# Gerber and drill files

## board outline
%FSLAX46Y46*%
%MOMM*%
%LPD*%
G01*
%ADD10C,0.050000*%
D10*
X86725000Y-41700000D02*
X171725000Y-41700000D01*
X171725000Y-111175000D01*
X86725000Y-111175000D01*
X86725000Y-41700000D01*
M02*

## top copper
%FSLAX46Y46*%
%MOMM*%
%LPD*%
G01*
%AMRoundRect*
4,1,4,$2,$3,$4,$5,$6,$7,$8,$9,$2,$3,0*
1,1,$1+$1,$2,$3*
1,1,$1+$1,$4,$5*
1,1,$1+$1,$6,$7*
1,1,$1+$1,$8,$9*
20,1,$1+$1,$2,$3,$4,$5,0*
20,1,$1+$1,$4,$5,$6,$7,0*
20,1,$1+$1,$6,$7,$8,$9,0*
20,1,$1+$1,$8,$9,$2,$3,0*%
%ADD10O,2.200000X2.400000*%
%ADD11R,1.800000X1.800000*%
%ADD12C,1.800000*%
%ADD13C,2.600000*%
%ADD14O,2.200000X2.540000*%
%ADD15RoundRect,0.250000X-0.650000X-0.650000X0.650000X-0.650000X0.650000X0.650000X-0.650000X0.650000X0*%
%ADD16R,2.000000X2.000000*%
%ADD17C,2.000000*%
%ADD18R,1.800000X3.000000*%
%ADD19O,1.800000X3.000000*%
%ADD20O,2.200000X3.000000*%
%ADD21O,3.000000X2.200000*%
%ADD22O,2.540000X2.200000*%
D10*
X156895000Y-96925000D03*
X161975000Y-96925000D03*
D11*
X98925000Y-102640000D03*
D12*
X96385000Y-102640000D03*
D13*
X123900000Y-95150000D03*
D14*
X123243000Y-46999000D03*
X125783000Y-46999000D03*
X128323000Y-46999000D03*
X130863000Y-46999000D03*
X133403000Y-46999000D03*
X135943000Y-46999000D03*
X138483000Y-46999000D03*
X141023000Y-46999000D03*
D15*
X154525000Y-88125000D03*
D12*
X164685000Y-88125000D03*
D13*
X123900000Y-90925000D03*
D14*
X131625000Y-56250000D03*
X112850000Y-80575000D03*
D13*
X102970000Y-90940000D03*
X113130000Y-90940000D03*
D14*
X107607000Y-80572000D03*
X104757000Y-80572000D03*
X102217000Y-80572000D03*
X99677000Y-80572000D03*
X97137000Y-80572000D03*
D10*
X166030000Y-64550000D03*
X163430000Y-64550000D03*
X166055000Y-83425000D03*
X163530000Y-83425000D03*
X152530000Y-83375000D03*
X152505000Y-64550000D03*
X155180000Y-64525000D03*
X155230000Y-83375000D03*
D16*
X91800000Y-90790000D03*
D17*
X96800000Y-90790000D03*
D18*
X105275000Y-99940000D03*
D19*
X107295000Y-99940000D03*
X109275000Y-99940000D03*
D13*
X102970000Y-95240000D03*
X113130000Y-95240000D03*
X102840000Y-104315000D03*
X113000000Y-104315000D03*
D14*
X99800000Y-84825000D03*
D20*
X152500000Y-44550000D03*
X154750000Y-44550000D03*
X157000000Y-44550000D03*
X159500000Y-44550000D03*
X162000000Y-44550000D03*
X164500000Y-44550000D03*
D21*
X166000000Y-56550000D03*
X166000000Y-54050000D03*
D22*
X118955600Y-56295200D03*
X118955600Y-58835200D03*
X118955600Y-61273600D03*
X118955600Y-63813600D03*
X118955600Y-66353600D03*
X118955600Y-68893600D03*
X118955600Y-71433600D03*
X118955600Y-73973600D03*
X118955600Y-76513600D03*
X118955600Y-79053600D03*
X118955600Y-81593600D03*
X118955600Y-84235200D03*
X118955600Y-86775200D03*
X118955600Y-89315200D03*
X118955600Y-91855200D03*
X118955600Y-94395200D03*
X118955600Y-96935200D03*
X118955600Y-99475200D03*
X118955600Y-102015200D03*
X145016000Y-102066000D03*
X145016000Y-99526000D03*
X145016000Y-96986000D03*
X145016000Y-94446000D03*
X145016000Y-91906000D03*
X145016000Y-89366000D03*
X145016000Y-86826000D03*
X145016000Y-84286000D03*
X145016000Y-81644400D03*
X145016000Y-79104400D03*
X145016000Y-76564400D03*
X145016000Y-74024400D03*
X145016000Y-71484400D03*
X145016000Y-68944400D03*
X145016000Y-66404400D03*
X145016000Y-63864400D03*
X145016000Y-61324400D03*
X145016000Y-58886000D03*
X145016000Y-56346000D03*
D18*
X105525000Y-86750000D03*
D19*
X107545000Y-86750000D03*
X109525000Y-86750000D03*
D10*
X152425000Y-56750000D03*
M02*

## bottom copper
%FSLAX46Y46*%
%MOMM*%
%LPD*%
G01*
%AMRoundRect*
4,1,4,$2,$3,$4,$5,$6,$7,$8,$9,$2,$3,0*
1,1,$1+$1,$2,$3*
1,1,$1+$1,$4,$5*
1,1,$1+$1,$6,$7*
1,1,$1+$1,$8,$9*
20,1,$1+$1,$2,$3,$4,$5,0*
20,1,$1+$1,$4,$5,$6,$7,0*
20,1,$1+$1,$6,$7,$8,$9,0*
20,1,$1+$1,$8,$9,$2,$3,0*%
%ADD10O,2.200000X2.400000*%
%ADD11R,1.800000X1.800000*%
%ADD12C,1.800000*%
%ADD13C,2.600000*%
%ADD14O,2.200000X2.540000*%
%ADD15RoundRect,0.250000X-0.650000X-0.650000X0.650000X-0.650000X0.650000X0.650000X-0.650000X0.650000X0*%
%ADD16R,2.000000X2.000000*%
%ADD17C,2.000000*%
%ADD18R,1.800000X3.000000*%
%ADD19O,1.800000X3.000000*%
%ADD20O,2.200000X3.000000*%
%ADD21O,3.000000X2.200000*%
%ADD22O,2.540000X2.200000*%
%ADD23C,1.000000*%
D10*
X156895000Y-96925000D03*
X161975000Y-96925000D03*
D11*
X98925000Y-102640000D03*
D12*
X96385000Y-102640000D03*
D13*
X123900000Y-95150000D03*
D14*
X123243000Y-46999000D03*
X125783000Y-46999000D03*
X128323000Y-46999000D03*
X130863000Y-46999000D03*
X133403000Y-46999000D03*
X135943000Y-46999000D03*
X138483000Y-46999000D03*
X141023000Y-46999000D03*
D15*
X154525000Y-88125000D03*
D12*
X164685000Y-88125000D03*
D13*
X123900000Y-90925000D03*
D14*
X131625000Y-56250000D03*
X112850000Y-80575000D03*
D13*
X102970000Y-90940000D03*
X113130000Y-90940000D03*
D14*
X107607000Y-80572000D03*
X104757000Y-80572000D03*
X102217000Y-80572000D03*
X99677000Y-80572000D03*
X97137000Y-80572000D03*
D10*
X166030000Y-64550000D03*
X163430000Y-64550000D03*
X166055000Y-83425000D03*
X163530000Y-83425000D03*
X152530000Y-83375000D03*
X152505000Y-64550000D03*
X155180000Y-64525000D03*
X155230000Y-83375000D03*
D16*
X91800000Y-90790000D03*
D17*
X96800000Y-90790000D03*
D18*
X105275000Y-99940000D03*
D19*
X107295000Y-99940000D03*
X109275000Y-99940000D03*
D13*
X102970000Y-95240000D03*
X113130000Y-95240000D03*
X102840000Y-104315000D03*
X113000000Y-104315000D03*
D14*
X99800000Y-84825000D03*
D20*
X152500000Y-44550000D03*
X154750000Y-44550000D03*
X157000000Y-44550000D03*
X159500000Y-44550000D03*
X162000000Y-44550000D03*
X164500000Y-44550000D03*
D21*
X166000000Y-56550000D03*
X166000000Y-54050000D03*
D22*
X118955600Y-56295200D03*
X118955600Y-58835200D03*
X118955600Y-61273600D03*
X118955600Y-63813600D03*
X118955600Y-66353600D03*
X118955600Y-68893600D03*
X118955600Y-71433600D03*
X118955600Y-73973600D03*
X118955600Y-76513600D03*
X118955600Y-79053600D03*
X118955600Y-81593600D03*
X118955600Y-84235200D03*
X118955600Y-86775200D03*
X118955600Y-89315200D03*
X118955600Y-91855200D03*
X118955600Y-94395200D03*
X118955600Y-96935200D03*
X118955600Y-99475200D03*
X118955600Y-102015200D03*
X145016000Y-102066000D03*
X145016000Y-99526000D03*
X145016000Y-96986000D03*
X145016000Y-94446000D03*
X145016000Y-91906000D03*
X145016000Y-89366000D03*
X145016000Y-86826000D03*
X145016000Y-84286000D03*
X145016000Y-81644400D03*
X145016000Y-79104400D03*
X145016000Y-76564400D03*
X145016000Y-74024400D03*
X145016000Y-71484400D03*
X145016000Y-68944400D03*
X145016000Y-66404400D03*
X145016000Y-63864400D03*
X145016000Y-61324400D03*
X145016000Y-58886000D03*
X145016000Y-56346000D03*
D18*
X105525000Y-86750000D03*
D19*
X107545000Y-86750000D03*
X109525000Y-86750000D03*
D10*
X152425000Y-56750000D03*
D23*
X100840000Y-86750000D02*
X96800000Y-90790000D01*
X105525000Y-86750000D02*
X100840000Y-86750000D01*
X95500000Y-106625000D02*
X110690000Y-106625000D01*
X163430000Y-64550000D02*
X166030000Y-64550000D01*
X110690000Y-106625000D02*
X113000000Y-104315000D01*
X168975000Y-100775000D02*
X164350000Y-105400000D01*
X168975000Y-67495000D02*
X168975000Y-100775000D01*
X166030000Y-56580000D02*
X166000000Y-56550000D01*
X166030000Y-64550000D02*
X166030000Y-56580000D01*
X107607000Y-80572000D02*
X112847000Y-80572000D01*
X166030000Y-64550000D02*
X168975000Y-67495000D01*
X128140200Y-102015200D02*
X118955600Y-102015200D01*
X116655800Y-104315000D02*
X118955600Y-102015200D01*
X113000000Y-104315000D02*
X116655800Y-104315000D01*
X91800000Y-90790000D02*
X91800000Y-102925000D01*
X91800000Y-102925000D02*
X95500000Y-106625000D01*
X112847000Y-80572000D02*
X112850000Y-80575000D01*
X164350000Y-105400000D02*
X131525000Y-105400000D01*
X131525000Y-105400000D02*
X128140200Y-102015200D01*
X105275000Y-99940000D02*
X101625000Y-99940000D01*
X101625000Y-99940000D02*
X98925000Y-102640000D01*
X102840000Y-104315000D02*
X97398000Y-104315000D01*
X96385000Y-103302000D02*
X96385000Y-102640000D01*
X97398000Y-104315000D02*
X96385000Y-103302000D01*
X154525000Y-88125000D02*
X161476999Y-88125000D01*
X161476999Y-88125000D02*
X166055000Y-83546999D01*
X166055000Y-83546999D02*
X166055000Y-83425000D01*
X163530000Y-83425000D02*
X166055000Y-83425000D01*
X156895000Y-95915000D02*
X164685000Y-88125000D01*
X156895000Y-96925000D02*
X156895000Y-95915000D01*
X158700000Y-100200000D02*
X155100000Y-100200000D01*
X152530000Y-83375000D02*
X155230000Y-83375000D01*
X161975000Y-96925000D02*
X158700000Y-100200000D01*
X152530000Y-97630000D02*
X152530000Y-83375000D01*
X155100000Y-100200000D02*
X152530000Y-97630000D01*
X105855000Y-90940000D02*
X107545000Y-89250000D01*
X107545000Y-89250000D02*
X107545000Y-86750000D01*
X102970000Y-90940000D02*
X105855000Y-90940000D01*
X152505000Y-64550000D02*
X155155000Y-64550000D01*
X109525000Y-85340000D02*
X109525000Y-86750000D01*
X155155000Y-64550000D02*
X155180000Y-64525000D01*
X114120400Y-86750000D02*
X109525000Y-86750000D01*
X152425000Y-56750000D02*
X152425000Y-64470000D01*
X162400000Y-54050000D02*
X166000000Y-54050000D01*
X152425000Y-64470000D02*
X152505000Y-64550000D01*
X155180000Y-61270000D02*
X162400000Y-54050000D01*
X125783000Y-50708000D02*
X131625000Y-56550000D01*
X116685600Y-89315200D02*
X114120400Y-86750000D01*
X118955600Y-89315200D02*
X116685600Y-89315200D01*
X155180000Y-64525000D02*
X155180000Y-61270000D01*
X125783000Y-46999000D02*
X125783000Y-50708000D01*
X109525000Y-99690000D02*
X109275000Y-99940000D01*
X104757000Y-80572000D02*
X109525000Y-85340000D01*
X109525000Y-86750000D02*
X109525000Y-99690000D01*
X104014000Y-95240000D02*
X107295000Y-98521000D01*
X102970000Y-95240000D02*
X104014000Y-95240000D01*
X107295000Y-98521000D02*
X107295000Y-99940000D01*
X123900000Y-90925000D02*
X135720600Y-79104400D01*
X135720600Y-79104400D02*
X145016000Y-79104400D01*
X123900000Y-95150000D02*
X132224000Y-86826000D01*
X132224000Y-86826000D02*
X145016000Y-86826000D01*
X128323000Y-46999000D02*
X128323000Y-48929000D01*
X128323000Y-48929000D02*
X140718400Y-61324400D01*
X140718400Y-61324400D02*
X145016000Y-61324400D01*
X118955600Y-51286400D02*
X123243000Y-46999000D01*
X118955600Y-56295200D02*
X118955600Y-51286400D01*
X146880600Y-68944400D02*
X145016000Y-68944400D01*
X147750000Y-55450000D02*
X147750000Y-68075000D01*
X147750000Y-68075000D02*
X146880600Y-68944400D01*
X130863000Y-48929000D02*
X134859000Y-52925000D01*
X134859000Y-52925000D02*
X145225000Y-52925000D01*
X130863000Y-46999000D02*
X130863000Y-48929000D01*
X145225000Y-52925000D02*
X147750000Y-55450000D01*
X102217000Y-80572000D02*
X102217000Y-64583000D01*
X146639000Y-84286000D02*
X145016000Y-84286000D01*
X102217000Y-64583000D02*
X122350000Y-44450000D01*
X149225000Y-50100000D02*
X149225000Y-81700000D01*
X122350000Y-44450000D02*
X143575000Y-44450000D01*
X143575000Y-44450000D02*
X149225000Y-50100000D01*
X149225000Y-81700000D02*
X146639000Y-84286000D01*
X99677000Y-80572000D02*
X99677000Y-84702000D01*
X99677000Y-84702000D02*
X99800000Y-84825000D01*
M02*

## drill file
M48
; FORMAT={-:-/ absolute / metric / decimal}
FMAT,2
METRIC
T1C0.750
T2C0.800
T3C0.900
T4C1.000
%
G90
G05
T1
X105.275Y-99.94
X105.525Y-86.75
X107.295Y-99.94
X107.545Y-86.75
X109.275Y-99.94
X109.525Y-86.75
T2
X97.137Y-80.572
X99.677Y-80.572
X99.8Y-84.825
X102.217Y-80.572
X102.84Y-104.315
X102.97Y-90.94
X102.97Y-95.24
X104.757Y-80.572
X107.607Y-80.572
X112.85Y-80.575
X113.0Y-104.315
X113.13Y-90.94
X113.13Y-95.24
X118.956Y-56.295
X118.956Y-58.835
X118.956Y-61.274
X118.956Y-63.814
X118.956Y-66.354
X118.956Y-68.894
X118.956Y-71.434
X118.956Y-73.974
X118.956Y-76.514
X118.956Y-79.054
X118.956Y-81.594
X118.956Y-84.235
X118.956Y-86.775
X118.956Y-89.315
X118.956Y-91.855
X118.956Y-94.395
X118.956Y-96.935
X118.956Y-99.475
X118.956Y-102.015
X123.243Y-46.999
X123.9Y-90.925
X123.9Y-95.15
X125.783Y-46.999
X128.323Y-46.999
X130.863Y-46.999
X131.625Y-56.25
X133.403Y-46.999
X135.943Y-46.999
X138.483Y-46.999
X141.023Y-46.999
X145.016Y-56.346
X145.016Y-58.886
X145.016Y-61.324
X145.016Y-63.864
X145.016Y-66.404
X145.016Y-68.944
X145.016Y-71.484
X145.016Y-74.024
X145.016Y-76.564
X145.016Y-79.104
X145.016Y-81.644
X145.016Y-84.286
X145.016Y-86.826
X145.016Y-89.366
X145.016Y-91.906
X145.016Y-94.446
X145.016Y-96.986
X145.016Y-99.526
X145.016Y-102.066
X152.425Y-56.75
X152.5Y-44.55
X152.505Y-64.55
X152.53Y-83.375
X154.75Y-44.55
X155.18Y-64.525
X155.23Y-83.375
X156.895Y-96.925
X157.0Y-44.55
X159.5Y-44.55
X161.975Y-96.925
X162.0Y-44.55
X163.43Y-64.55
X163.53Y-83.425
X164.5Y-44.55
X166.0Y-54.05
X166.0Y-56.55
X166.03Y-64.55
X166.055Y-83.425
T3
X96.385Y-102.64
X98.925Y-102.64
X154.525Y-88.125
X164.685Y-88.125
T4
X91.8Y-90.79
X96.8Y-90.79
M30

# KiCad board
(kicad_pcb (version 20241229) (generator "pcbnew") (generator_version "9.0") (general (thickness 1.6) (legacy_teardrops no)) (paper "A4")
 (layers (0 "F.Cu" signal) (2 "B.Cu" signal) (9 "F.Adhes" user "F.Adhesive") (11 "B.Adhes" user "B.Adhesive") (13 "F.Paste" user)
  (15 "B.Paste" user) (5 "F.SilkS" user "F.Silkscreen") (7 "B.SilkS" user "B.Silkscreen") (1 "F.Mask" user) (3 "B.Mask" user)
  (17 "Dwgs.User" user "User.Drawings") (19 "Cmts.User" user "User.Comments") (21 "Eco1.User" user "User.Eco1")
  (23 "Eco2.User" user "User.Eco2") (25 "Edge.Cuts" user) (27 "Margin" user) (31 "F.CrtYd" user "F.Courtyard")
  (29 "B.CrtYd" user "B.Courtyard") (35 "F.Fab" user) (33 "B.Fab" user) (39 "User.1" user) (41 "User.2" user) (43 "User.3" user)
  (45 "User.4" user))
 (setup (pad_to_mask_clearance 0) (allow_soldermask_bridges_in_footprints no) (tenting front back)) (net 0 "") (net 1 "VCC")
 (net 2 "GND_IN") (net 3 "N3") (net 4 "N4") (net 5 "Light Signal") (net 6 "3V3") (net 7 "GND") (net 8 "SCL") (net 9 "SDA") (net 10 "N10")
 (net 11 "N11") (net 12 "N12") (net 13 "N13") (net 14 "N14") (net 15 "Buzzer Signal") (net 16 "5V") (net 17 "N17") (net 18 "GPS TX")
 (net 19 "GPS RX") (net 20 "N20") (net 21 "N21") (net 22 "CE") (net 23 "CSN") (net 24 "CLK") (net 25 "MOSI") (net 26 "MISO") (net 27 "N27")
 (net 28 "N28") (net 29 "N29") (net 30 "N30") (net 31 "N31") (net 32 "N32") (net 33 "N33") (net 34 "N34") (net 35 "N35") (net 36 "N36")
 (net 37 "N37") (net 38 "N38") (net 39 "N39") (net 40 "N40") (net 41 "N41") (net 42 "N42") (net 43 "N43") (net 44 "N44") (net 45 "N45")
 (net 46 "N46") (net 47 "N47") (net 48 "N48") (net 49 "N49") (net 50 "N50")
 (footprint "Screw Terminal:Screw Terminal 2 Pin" (layer "F.Cu") (at 154.355 93.075)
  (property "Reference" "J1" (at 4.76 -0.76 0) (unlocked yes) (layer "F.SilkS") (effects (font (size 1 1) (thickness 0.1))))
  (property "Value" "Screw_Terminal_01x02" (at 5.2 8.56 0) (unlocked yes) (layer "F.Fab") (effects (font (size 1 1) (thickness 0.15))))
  (pad "1" thru_hole oval (at 2.54 3.85 90) (size 2.4 2.2) (drill 0.8) (layers "*.Cu" "*.Mask") (remove_unused_layers no) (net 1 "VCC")
   (thermal_bridge_angle 45))
  (pad "2" thru_hole oval (at 7.62 3.85 90) (size 2.4 2.2) (drill 0.8) (layers "*.Cu" "*.Mask") (remove_unused_layers no) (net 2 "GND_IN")
   (thermal_bridge_angle 45)))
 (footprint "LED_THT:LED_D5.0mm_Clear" (layer "F.Cu") (at 98.925 102.64 180)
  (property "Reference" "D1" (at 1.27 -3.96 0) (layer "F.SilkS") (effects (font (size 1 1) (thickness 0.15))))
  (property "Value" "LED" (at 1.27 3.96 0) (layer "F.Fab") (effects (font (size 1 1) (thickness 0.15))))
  (pad "1" thru_hole rect (at 0 0 180) (size 1.8 1.8) (drill 0.9) (layers "*.Cu" "*.Mask") (remove_unused_layers no) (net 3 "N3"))
  (pad "2" thru_hole circle (at 2.54 0 180) (size 1.8 1.8) (drill 0.9) (layers "*.Cu" "*.Mask") (remove_unused_layers no) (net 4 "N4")))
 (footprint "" (layer "F.Cu") (at 123.9 95.15)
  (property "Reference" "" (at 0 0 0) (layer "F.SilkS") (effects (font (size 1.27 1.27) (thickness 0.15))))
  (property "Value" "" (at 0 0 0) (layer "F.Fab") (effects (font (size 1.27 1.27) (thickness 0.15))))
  (pad "2" thru_hole circle (at 0 0) (size 2.6 2.6) (drill 0.8) (layers "*.Cu" "*.Mask") (remove_unused_layers no) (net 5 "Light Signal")))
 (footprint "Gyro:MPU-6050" (layer "F.Cu") (at 121.719 32.775)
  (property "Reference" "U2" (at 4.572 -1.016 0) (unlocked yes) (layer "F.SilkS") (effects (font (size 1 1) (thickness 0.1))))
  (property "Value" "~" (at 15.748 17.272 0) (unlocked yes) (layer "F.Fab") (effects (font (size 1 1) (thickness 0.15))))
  (pad "1" thru_hole oval (at 1.524 14.224 90) (size 2.54 2.2) (drill 0.8) (layers "*.Cu" "*.Mask") (remove_unused_layers no) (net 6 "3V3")
   (thermal_bridge_angle 45))
  (pad "2" thru_hole oval (at 4.064 14.224 90) (size 2.54 2.2) (drill 0.8) (layers "*.Cu" "*.Mask") (remove_unused_layers no) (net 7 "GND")
   (thermal_bridge_angle 45))
  (pad "3" thru_hole oval (at 6.604 14.224 90) (size 2.54 2.2) (drill 0.8) (layers "*.Cu" "*.Mask") (remove_unused_layers no) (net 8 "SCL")
   (thermal_bridge_angle 45))
  (pad "4" thru_hole oval (at 9.144 14.224 90) (size 2.54 2.2) (drill 0.8) (layers "*.Cu" "*.Mask") (remove_unused_layers no) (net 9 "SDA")
   (thermal_bridge_angle 45))
  (pad "5" thru_hole oval (at 11.684 14.224 90) (size 2.54 2.2) (drill 0.8) (layers "*.Cu" "*.Mask") (remove_unused_layers no)
   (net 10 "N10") (thermal_bridge_angle 45))
  (pad "6" thru_hole oval (at 14.224 14.224 90) (size 2.54 2.2) (drill 0.8) (layers "*.Cu" "*.Mask") (remove_unused_layers no)
   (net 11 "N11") (thermal_bridge_angle 45))
  (pad "7" thru_hole oval (at 16.764 14.224 90) (size 2.54 2.2) (drill 0.8) (layers "*.Cu" "*.Mask") (remove_unused_layers no)
   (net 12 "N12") (thermal_bridge_angle 45))
  (pad "8" thru_hole oval (at 19.304 14.224 90) (size 2.54 2.2) (drill 0.8) (layers "*.Cu" "*.Mask") (remove_unused_layers no)
   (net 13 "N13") (thermal_bridge_angle 45)))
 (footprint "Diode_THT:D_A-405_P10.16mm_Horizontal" (layer "F.Cu") (at 154.525 88.125)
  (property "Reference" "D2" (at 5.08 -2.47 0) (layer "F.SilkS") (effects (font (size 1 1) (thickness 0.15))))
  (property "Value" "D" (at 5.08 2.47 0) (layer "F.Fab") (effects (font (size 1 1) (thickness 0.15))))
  (pad "1" thru_hole roundrect (at 0 0) (size 1.8 1.8) (drill 0.9) (layers "*.Cu" "*.Mask") (remove_unused_layers no)
   (roundrect_rratio 0.138889) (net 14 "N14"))
  (pad "2" thru_hole circle (at 10.16 0) (size 1.8 1.8) (drill 0.9) (layers "*.Cu" "*.Mask") (remove_unused_layers no) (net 1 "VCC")))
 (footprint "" (layer "F.Cu") (at 123.9 90.925)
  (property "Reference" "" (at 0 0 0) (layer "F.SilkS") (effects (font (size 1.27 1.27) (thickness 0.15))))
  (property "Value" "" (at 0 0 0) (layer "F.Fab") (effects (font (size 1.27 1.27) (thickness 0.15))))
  (pad "2" thru_hole circle (at 0 0) (size 2.6 2.6) (drill 0.8) (layers "*.Cu" "*.Mask") (remove_unused_layers no) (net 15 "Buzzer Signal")))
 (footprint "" (layer "F.Cu") (at 131.625 56.25)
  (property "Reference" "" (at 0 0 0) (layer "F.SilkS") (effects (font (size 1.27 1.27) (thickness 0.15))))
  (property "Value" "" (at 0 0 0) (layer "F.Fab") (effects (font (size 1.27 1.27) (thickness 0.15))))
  (pad "2" thru_hole oval (at 0 0 90) (size 2.54 2.2) (drill 0.8) (layers "*.Cu" "*.Mask") (remove_unused_layers no) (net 7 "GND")
   (thermal_bridge_angle 45)))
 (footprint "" (layer "F.Cu") (at 112.85 80.575)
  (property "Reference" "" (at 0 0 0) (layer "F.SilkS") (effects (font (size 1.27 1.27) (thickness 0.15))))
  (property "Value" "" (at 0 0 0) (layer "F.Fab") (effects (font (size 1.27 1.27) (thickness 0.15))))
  (pad "1" thru_hole oval (at 0 0 270) (size 2.54 2.2) (drill 0.8) (layers "*.Cu" "*.Mask") (remove_unused_layers no) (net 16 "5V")
   (thermal_bridge_angle 45)))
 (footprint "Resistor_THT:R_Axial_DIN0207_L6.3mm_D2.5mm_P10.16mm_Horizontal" (layer "F.Cu") (at 102.97 90.94)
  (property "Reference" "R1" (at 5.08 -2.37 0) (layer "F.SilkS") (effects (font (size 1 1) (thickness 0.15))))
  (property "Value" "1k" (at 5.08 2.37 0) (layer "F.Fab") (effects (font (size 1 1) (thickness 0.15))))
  (pad "1" thru_hole circle (at 0 0) (size 2.6 2.6) (drill 0.8) (layers "*.Cu" "*.Mask") (remove_unused_layers no) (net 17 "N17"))
  (pad "2" thru_hole circle (at 10.16 0) (size 2.6 2.6) (drill 0.8) (layers "*.Cu" "*.Mask") (remove_unused_layers no)
   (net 15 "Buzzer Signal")))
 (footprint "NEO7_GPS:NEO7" (layer "F.Cu") (at 115.425 30.153 -90)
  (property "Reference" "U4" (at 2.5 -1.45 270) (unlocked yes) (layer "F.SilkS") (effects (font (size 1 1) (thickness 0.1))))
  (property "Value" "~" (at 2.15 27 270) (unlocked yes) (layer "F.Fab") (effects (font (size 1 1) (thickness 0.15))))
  (pad "1" thru_hole oval (at 50.419 7.818 270) (size 2.54 2.2) (drill 0.8) (layers "*.Cu" "*.Mask") (remove_unused_layers no) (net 16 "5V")
   (thermal_bridge_angle 45))
  (pad "2" thru_hole oval (at 50.419 10.668 270) (size 2.54 2.2) (drill 0.8) (layers "*.Cu" "*.Mask") (remove_unused_layers no)
   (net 7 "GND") (thermal_bridge_angle 45))
  (pad "3" thru_hole oval (at 50.419 13.208 270) (size 2.54 2.2) (drill 0.8) (layers "*.Cu" "*.Mask") (remove_unused_layers no)
   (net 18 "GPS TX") (thermal_bridge_angle 45))
  (pad "4" thru_hole oval (at 50.419 15.748 270) (size 2.54 2.2) (drill 0.8) (layers "*.Cu" "*.Mask") (remove_unused_layers no)
   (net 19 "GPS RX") (thermal_bridge_angle 45))
  (pad "5" thru_hole oval (at 50.419 18.288 270) (size 2.54 2.2) (drill 0.8) (layers "*.Cu" "*.Mask") (remove_unused_layers no)
   (thermal_bridge_angle 45)))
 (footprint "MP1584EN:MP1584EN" (layer "F.Cu") (at 168.33 62.45 -90)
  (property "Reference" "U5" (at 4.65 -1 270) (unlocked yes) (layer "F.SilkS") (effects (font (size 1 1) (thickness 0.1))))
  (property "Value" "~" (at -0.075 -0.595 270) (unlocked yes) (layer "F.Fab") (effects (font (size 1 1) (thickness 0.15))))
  (pad "1" thru_hole oval (at 2.1 2.3 270) (size 2.4 2.2) (drill 0.8) (layers "*.Cu" "*.Mask") (remove_unused_layers no) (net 16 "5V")
   (thermal_bridge_angle 45))
  (pad "2" thru_hole oval (at 2.1 4.9 270) (size 2.4 2.2) (drill 0.8) (layers "*.Cu" "*.Mask") (remove_unused_layers no) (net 16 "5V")
   (thermal_bridge_angle 45))
  (pad "3" thru_hole oval (at 20.975 2.275 270) (size 2.4 2.2) (drill 0.8) (layers "*.Cu" "*.Mask") (remove_unused_layers no) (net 14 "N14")
   (thermal_bridge_angle 45))
  (pad "4" thru_hole oval (at 20.975 4.8 270) (size 2.4 2.2) (drill 0.8) (layers "*.Cu" "*.Mask") (remove_unused_layers no) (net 14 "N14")
   (thermal_bridge_angle 45))
  (pad "5" thru_hole oval (at 20.925 15.8 270) (size 2.4 2.2) (drill 0.8) (layers "*.Cu" "*.Mask") (remove_unused_layers no)
   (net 2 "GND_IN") (thermal_bridge_angle 45))
  (pad "6" thru_hole oval (at 2.1 15.825 270) (size 2.4 2.2) (drill 0.8) (layers "*.Cu" "*.Mask") (remove_unused_layers no) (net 7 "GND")
   (thermal_bridge_angle 45))
  (pad "7" thru_hole oval (at 2.075 13.15 270) (size 2.4 2.2) (drill 0.8) (layers "*.Cu" "*.Mask") (remove_unused_layers no) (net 7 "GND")
   (thermal_bridge_angle 45))
  (pad "8" thru_hole oval (at 20.925 13.1 270) (size 2.4 2.2) (drill 0.8) (layers "*.Cu" "*.Mask") (remove_unused_layers no)
   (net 2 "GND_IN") (thermal_bridge_angle 45)))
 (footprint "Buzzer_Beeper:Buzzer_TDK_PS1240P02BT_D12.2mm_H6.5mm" (layer "F.Cu") (at 91.8 90.79)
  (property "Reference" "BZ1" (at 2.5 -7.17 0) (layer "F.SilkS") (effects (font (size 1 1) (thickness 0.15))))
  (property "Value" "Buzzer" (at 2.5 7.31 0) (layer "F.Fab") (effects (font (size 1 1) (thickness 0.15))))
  (pad "1" thru_hole rect (at 0 0) (size 2 2) (drill 1) (layers "*.Cu" "*.Mask") (remove_unused_layers no) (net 16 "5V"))
  (pad "2" thru_hole circle (at 5 0) (size 2 2) (drill 1) (layers "*.Cu" "*.Mask") (remove_unused_layers no) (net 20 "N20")))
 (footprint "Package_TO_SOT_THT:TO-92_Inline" (layer "F.Cu") (at 106.025 99.94)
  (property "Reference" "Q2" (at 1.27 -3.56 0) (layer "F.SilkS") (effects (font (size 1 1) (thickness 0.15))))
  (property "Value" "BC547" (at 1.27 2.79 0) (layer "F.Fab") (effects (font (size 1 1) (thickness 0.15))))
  (pad "1" thru_hole rect (at -0.75 0) (size 1.8 3) (drill 0.75) (layers "*.Cu" "*.Mask") (remove_unused_layers no) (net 3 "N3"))
  (pad "2" thru_hole oval (at 1.27 0) (size 1.8 3) (drill 0.75) (layers "*.Cu" "*.Mask") (remove_unused_layers no) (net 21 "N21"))
  (pad "3" thru_hole oval (at 3.25 0) (size 1.8 3) (drill 0.75) (layers "*.Cu" "*.Mask") (remove_unused_layers no) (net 7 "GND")))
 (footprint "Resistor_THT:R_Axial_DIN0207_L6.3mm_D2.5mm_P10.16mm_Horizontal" (layer "F.Cu") (at 102.97 95.24)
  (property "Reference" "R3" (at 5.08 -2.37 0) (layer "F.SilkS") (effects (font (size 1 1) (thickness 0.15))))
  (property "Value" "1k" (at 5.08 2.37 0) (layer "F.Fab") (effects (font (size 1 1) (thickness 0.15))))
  (pad "1" thru_hole circle (at 0 0) (size 2.6 2.6) (drill 0.8) (layers "*.Cu" "*.Mask") (remove_unused_layers no) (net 21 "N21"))
  (pad "2" thru_hole circle (at 10.16 0) (size 2.6 2.6) (drill 0.8) (layers "*.Cu" "*.Mask") (remove_unused_layers no)
   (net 5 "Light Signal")))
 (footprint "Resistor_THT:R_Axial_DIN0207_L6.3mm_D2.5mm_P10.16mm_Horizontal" (layer "F.Cu") (at 102.84 104.315)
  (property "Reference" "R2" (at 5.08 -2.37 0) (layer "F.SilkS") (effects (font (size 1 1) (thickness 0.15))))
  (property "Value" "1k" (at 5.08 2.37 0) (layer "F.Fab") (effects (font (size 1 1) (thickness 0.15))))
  (pad "1" thru_hole circle (at 0 0) (size 2.6 2.6) (drill 0.8) (layers "*.Cu" "*.Mask") (remove_unused_layers no) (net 4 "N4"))
  (pad "2" thru_hole circle (at 10.16 0) (size 2.6 2.6) (drill 0.8) (layers "*.Cu" "*.Mask") (remove_unused_layers no) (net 16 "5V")))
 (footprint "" (layer "F.Cu") (at 99.8 84.825)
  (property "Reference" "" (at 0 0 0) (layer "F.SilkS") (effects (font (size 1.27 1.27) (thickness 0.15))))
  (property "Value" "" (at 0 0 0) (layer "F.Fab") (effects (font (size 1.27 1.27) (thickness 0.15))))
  (pad "4" thru_hole oval (at 0 0 270) (size 2.54 2.2) (drill 0.8) (layers "*.Cu" "*.Mask") (remove_unused_layers no) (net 19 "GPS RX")
   (thermal_bridge_angle 45)))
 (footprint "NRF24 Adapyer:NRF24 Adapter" (layer "F.Cu") (at 158 47.8 90)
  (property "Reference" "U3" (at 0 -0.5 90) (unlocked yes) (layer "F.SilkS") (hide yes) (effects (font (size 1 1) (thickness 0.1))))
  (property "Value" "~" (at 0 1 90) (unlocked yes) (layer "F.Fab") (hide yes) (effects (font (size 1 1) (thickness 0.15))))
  (pad "1" thru_hole oval (at 3.25 -5.5 90) (size 3 2.2) (drill 0.8) (layers "*.Cu" "*.Mask") (remove_unused_layers no) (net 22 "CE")
   (thermal_bridge_angle 45))
  (pad "2" thru_hole oval (at 3.25 -3.25 90) (size 3 2.2) (drill 0.8) (layers "*.Cu" "*.Mask") (remove_unused_layers no) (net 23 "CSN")
   (thermal_bridge_angle 45))
  (pad "3" thru_hole oval (at 3.25 -1 90) (size 3 2.2) (drill 0.8) (layers "*.Cu" "*.Mask") (remove_unused_layers no) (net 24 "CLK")
   (thermal_bridge_angle 45))
  (pad "4" thru_hole oval (at 3.25 1.5 90) (size 3 2.2) (drill 0.8) (layers "*.Cu" "*.Mask") (remove_unused_layers no) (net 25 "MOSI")
   (thermal_bridge_angle 45))
  (pad "5" thru_hole oval (at 3.25 4 90) (size 3 2.2) (drill 0.8) (layers "*.Cu" "*.Mask") (remove_unused_layers no) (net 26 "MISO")
   (thermal_bridge_angle 45))
  (pad "6" thru_hole oval (at 3.25 6.5 90) (size 3 2.2) (drill 0.8) (layers "*.Cu" "*.Mask") (remove_unused_layers no) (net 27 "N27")
   (thermal_bridge_angle 45))
  (pad "7" thru_hole oval (at -8.75 8 90) (size 2.2 3) (drill 0.8) (layers "*.Cu" "*.Mask") (remove_unused_layers no) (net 16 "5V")
   (thermal_bridge_angle 45))
  (pad "8" thru_hole oval (at -6.25 8 90) (size 2.2 3) (drill 0.8) (layers "*.Cu" "*.Mask") (remove_unused_layers no) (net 7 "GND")
   (thermal_bridge_angle 45))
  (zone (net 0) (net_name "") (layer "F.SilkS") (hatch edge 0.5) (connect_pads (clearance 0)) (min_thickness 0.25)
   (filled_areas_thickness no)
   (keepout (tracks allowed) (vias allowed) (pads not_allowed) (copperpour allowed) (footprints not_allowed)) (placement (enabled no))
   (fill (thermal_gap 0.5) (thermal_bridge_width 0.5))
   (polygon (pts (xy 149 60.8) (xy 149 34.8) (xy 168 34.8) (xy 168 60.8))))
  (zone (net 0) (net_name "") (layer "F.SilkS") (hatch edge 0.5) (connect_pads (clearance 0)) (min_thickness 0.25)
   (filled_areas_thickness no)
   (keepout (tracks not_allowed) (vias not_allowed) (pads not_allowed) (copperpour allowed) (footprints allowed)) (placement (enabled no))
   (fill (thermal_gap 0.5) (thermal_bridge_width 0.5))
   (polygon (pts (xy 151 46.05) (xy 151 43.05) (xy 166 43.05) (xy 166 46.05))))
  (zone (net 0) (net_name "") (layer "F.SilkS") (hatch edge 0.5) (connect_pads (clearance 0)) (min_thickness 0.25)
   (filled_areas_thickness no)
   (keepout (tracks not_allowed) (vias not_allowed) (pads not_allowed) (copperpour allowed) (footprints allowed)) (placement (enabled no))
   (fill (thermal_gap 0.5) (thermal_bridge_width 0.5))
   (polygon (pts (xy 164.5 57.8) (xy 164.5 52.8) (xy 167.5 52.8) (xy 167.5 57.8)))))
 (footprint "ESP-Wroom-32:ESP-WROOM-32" (layer "F.Cu") (at 119.616 51.9264)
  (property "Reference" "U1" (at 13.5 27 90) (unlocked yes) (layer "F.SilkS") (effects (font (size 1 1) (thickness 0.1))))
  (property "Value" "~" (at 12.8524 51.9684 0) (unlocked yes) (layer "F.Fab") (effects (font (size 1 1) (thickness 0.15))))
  (pad "1" thru_hole oval (at -0.6604 4.3688) (size 2.54 2.2) (drill 0.8) (layers "*.Cu" "*.Mask") (remove_unused_layers no) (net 6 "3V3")
   (thermal_bridge_angle 45))
  (pad "2" thru_hole oval (at -0.6604 6.9088) (size 2.54 2.2) (drill 0.8) (layers "*.Cu" "*.Mask") (remove_unused_layers no) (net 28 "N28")
   (thermal_bridge_angle 45))
  (pad "3" thru_hole oval (at -0.6604 9.3472) (size 2.54 2.2) (drill 0.8) (layers "*.Cu" "*.Mask") (remove_unused_layers no) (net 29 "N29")
   (thermal_bridge_angle 45))
  (pad "4" thru_hole oval (at -0.6604 11.8872) (size 2.54 2.2) (drill 0.8) (layers "*.Cu" "*.Mask") (remove_unused_layers no) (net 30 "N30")
   (thermal_bridge_angle 45))
  (pad "5" thru_hole oval (at -0.6604 14.4272) (size 2.54 2.2) (drill 0.8) (layers "*.Cu" "*.Mask") (remove_unused_layers no) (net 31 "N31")
   (thermal_bridge_angle 45))
  (pad "6" thru_hole oval (at -0.6604 16.9672) (size 2.54 2.2) (drill 0.8) (layers "*.Cu" "*.Mask") (remove_unused_layers no) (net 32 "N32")
   (thermal_bridge_angle 45))
  (pad "7" thru_hole oval (at -0.6604 19.5072) (size 2.54 2.2) (drill 0.8) (layers "*.Cu" "*.Mask") (remove_unused_layers no) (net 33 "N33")
   (thermal_bridge_angle 45))
  (pad "8" thru_hole oval (at -0.6604 22.0472) (size 2.54 2.2) (drill 0.8) (layers "*.Cu" "*.Mask") (remove_unused_layers no) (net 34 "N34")
   (thermal_bridge_angle 45))
  (pad "9" thru_hole oval (at -0.6604 24.5872) (size 2.54 2.2) (drill 0.8) (layers "*.Cu" "*.Mask") (remove_unused_layers no) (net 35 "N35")
   (thermal_bridge_angle 45))
  (pad "10" thru_hole oval (at -0.6604 27.1272) (size 2.54 2.2) (drill 0.8) (layers "*.Cu" "*.Mask") (remove_unused_layers no)
   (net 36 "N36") (thermal_bridge_angle 45))
  (pad "11" thru_hole oval (at -0.6604 29.6672) (size 2.54 2.2) (drill 0.8) (layers "*.Cu" "*.Mask") (remove_unused_layers no)
   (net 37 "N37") (thermal_bridge_angle 45))
  (pad "12" thru_hole oval (at -0.6604 32.3088) (size 2.54 2.2) (drill 0.8) (layers "*.Cu" "*.Mask") (remove_unused_layers no)
   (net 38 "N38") (thermal_bridge_angle 45))
  (pad "13" thru_hole oval (at -0.6604 34.8488) (size 2.54 2.2) (drill 0.8) (layers "*.Cu" "*.Mask") (remove_unused_layers no)
   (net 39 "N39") (thermal_bridge_angle 45))
  (pad "14" thru_hole oval (at -0.6604 37.3888) (size 2.54 2.2) (drill 0.8) (layers "*.Cu" "*.Mask") (remove_unused_layers no) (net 7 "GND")
   (thermal_bridge_angle 45))
  (pad "15" thru_hole oval (at -0.6604 39.9288) (size 2.54 2.2) (drill 0.8) (layers "*.Cu" "*.Mask") (remove_unused_layers no)
   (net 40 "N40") (thermal_bridge_angle 45))
  (pad "16" thru_hole oval (at -0.6604 42.4688) (size 2.54 2.2) (drill 0.8) (layers "*.Cu" "*.Mask") (remove_unused_layers no)
   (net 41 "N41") (thermal_bridge_angle 45))
  (pad "17" thru_hole oval (at -0.6604 45.0088) (size 2.54 2.2) (drill 0.8) (layers "*.Cu" "*.Mask") (remove_unused_layers no)
   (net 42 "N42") (thermal_bridge_angle 45))
  (pad "18" thru_hole oval (at -0.6604 47.5488) (size 2.54 2.2) (drill 0.8) (layers "*.Cu" "*.Mask") (remove_unused_layers no)
   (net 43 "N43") (thermal_bridge_angle 45))
  (pad "19" thru_hole oval (at -0.6604 50.0888) (size 2.54 2.2) (drill 0.8) (layers "*.Cu" "*.Mask") (remove_unused_layers no) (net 16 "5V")
   (thermal_bridge_angle 45))
  (pad "20" thru_hole oval (at 25.4 50.1396) (size 2.54 2.2) (drill 0.8) (layers "*.Cu" "*.Mask") (remove_unused_layers no) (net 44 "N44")
   (thermal_bridge_angle 45))
  (pad "21" thru_hole oval (at 25.4 47.5996) (size 2.54 2.2) (drill 0.8) (layers "*.Cu" "*.Mask") (remove_unused_layers no) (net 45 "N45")
   (thermal_bridge_angle 45))
  (pad "22" thru_hole oval (at 25.4 45.0596) (size 2.54 2.2) (drill 0.8) (layers "*.Cu" "*.Mask") (remove_unused_layers no) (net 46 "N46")
   (thermal_bridge_angle 45))
  (pad "23" thru_hole oval (at 25.4 42.5196) (size 2.54 2.2) (drill 0.8) (layers "*.Cu" "*.Mask") (remove_unused_layers no) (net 23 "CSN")
   (thermal_bridge_angle 45))
  (pad "24" thru_hole oval (at 25.4 39.9796) (size 2.54 2.2) (drill 0.8) (layers "*.Cu" "*.Mask") (remove_unused_layers no) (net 22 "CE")
   (thermal_bridge_angle 45))
  (pad "25" thru_hole oval (at 25.4 37.4396) (size 2.54 2.2) (drill 0.8) (layers "*.Cu" "*.Mask") (remove_unused_layers no) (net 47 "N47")
   (thermal_bridge_angle 45))
  (pad "26" thru_hole oval (at 25.4 34.8996) (size 2.54 2.2) (drill 0.8) (layers "*.Cu" "*.Mask") (remove_unused_layers no)
   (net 5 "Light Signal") (thermal_bridge_angle 45))
  (pad "27" thru_hole oval (at 25.4 32.3596) (size 2.54 2.2) (drill 0.8) (layers "*.Cu" "*.Mask") (remove_unused_layers no)
   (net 18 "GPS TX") (thermal_bridge_angle 45))
  (pad "28" thru_hole oval (at 25.4 29.718) (size 2.54 2.2) (drill 0.8) (layers "*.Cu" "*.Mask") (remove_unused_layers no) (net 19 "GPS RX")
   (thermal_bridge_angle 45))
  (pad "29" thru_hole oval (at 25.4 27.178) (size 2.54 2.2) (drill 0.8) (layers "*.Cu" "*.Mask") (remove_unused_layers no)
   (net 15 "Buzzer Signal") (thermal_bridge_angle 45))
  (pad "30" thru_hole oval (at 25.4 24.638) (size 2.54 2.2) (drill 0.8) (layers "*.Cu" "*.Mask") (remove_unused_layers no) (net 24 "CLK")
   (thermal_bridge_angle 45))
  (pad "31" thru_hole oval (at 25.4 22.098) (size 2.54 2.2) (drill 0.8) (layers "*.Cu" "*.Mask") (remove_unused_layers no) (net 26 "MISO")
   (thermal_bridge_angle 45))
  (pad "32" thru_hole oval (at 25.4 19.558) (size 2.54 2.2) (drill 0.8) (layers "*.Cu" "*.Mask") (remove_unused_layers no) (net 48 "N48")
   (thermal_bridge_angle 45))
  (pad "33" thru_hole oval (at 25.4 17.018) (size 2.54 2.2) (drill 0.8) (layers "*.Cu" "*.Mask") (remove_unused_layers no) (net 9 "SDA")
   (thermal_bridge_angle 45))
  (pad "34" thru_hole oval (at 25.4 14.478) (size 2.54 2.2) (drill 0.8) (layers "*.Cu" "*.Mask") (remove_unused_layers no) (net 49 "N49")
   (thermal_bridge_angle 45))
  (pad "35" thru_hole oval (at 25.4 11.938) (size 2.54 2.2) (drill 0.8) (layers "*.Cu" "*.Mask") (remove_unused_layers no) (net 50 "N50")
   (thermal_bridge_angle 45))
  (pad "36" thru_hole oval (at 25.4 9.398) (size 2.54 2.2) (drill 0.8) (layers "*.Cu" "*.Mask") (remove_unused_layers no) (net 8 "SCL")
   (thermal_bridge_angle 45))
  (pad "37" thru_hole oval (at 25.4 6.9596) (size 2.54 2.2) (drill 0.8) (layers "*.Cu" "*.Mask") (remove_unused_layers no) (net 25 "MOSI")
   (thermal_bridge_angle 45))
  (pad "38" thru_hole oval (at 25.4 4.4196) (size 2.54 2.2) (drill 0.8) (layers "*.Cu" "*.Mask") (remove_unused_layers no) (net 7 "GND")
   (thermal_bridge_angle 45)))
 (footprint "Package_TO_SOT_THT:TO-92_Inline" (layer "F.Cu") (at 106.275 86.75)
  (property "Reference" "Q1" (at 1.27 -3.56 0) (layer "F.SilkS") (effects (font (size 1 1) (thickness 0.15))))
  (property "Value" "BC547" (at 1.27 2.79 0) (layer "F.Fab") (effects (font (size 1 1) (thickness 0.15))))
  (pad "1" thru_hole rect (at -0.75 0) (size 1.8 3) (drill 0.75) (layers "*.Cu" "*.Mask") (remove_unused_layers no) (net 20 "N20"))
  (pad "2" thru_hole oval (at 1.27 0) (size 1.8 3) (drill 0.75) (layers "*.Cu" "*.Mask") (remove_unused_layers no) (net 17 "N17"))
  (pad "3" thru_hole oval (at 3.25 0) (size 1.8 3) (drill 0.75) (layers "*.Cu" "*.Mask") (remove_unused_layers no) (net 7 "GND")))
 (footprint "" (layer "F.Cu") (at 152.425 56.75)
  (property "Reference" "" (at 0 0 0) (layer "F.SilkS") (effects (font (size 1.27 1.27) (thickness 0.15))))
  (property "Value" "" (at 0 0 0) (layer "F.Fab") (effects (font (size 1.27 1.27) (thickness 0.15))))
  (pad "6" thru_hole oval (at 0 0 270) (size 2.4 2.2) (drill 0.8) (layers "*.Cu" "*.Mask") (remove_unused_layers no) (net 7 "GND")
   (thermal_bridge_angle 45)))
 (gr_rect (start 86.725 41.7) (end 171.725 111.175) (stroke (width 0.05) (type solid)) (fill no) (layer "Edge.Cuts"))
 (segment (start 100.84 86.75) (end 96.8 90.79) (width 1) (layer "B.Cu") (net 20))
 (segment (start 105.525 86.75) (end 100.84 86.75) (width 1) (layer "B.Cu") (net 20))
 (segment (start 95.5 106.625) (end 110.69 106.625) (width 1) (layer "B.Cu") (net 16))
 (segment (start 163.43 64.55) (end 166.03 64.55) (width 1) (layer "B.Cu") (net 16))
 (segment (start 110.69 106.625) (end 113 104.315) (width 1) (layer "B.Cu") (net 16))
 (segment (start 168.975 100.775) (end 164.35 105.4) (width 1) (layer "B.Cu") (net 16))
 (segment (start 168.975 67.495) (end 168.975 100.775) (width 1) (layer "B.Cu") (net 16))
 (segment (start 166.03 56.58) (end 166 56.55) (width 1) (layer "B.Cu") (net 16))
 (segment (start 166.03 64.55) (end 166.03 56.58) (width 1) (layer "B.Cu") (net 16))
 (segment (start 107.607 80.572) (end 112.847 80.572) (width 1) (layer "B.Cu") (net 16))
 (segment (start 166.03 64.55) (end 168.975 67.495) (width 1) (layer "B.Cu") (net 16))
 (segment (start 128.1402 102.0152) (end 118.9556 102.0152) (width 1) (layer "B.Cu") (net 16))
 (segment (start 116.6558 104.315) (end 118.9556 102.0152) (width 1) (layer "B.Cu") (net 16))
 (segment (start 113 104.315) (end 116.6558 104.315) (width 1) (layer "B.Cu") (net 16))
 (segment (start 91.8 90.79) (end 91.8 102.925) (width 1) (layer "B.Cu") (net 16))
 (segment (start 91.8 102.925) (end 95.5 106.625) (width 1) (layer "B.Cu") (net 16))
 (segment (start 112.847 80.572) (end 112.85 80.575) (width 1) (layer "B.Cu") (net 16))
 (segment (start 164.35 105.4) (end 131.525 105.4) (width 1) (layer "B.Cu") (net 16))
 (segment (start 131.525 105.4) (end 128.1402 102.0152) (width 1) (layer "B.Cu") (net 16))
 (segment (start 105.275 99.94) (end 101.625 99.94) (width 1) (layer "B.Cu") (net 3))
 (segment (start 101.625 99.94) (end 98.925 102.64) (width 1) (layer "B.Cu") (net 3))
 (segment (start 102.84 104.315) (end 97.398 104.315) (width 1) (layer "B.Cu") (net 4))
 (segment (start 96.385 103.302) (end 96.385 102.64) (width 1) (layer "B.Cu") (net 4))
 (segment (start 97.398 104.315) (end 96.385 103.302) (width 1) (layer "B.Cu") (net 4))
 (segment (start 154.525 88.125) (end 161.476999 88.125) (width 1) (layer "B.Cu") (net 14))
 (segment (start 161.476999 88.125) (end 166.055 83.546999) (width 1) (layer "B.Cu") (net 14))
 (segment (start 166.055 83.546999) (end 166.055 83.425) (width 1) (layer "B.Cu") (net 14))
 (segment (start 163.53 83.425) (end 166.055 83.425) (width 1) (layer "B.Cu") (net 14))
 (segment (start 156.895 95.915) (end 164.685 88.125) (width 1) (layer "B.Cu") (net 1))
 (segment (start 156.895 96.925) (end 156.895 95.915) (width 1) (layer "B.Cu") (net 1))
 (segment (start 158.7 100.2) (end 155.1 100.2) (width 1) (layer "B.Cu") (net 2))
 (segment (start 152.53 83.375) (end 155.23 83.375) (width 1) (layer "B.Cu") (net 2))
 (segment (start 161.975 96.925) (end 158.7 100.2) (width 1) (layer "B.Cu") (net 2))
 (segment (start 152.53 97.63) (end 152.53 83.375) (width 1) (layer "B.Cu") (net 2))
 (segment (start 155.1 100.2) (end 152.53 97.63) (width 1) (layer "B.Cu") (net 2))
 (segment (start 105.855 90.94) (end 107.545 89.25) (width 1) (layer "B.Cu") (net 17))
 (segment (start 107.545 89.25) (end 107.545 86.75) (width 1) (layer "B.Cu") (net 17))
 (segment (start 102.97 90.94) (end 105.855 90.94) (width 1) (layer "B.Cu") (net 17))
 (segment (start 152.505 64.55) (end 155.155 64.55) (width 1) (layer "B.Cu") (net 7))
 (segment (start 109.525 85.34) (end 109.525 86.75) (width 1) (layer "B.Cu") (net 7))
 (segment (start 155.155 64.55) (end 155.18 64.525) (width 1) (layer "B.Cu") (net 7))
 (segment (start 114.1204 86.75) (end 109.525 86.75) (width 1) (layer "B.Cu") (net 7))
 (segment (start 152.425 56.75) (end 152.425 64.47) (width 1) (layer "B.Cu") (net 7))
 (segment (start 162.4 54.05) (end 166 54.05) (width 1) (layer "B.Cu") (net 7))
 (segment (start 152.425 64.47) (end 152.505 64.55) (width 1) (layer "B.Cu") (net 7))
 (segment (start 155.18 61.27) (end 162.4 54.05) (width 1) (layer "B.Cu") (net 7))
 (segment (start 125.783 50.708) (end 131.625 56.55) (width 1) (layer "B.Cu") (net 7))
 (segment (start 116.6856 89.3152) (end 114.1204 86.75) (width 1) (layer "B.Cu") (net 7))
 (segment (start 118.9556 89.3152) (end 116.6856 89.3152) (width 1) (layer "B.Cu") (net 7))
 (segment (start 155.18 64.525) (end 155.18 61.27) (width 1) (layer "B.Cu") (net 7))
 (segment (start 125.783 46.999) (end 125.783 50.708) (width 1) (layer "B.Cu") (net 7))
 (segment (start 109.525 99.69) (end 109.275 99.94) (width 1) (layer "B.Cu") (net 7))
 (segment (start 104.757 80.572) (end 109.525 85.34) (width 1) (layer "B.Cu") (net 7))
 (segment (start 109.525 86.75) (end 109.525 99.69) (width 1) (layer "B.Cu") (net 7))
 (segment (start 104.014 95.24) (end 107.295 98.521) (width 1) (layer "B.Cu") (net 21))
 (segment (start 102.97 95.24) (end 104.014 95.24) (width 1) (layer "B.Cu") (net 21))
 (segment (start 107.295 98.521) (end 107.295 99.94) (width 1) (layer "B.Cu") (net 21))
 (segment (start 123.9 90.925) (end 135.7206 79.1044) (width 1) (layer "B.Cu") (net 15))
 (segment (start 135.7206 79.1044) (end 145.016 79.1044) (width 1) (layer "B.Cu") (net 15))
 (segment (start 123.9 95.15) (end 132.224 86.826) (width 1) (layer "B.Cu") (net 5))
 (segment (start 132.224 86.826) (end 145.016 86.826) (width 1) (layer "B.Cu") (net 5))
 (segment (start 128.323 46.999) (end 128.323 48.929) (width 1) (layer "B.Cu") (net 8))
 (segment (start 128.323 48.929) (end 140.7184 61.3244) (width 1) (layer "B.Cu") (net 8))
 (segment (start 140.7184 61.3244) (end 145.016 61.3244) (width 1) (layer "B.Cu") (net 8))
 (segment (start 118.9556 51.2864) (end 123.243 46.999) (width 1) (layer "B.Cu") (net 6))
 (segment (start 118.9556 56.2952) (end 118.9556 51.2864) (width 1) (layer "B.Cu") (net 6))
 (segment (start 146.8806 68.9444) (end 145.016 68.9444) (width 1) (layer "B.Cu") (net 9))
 (segment (start 147.75 55.45) (end 147.75 68.075) (width 1) (layer "B.Cu") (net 9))
 (segment (start 147.75 68.075) (end 146.8806 68.9444) (width 1) (layer "B.Cu") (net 9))
 (segment (start 130.863 48.929) (end 134.859 52.925) (width 1) (layer "B.Cu") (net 9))
 (segment (start 134.859 52.925) (end 145.225 52.925) (width 1) (layer "B.Cu") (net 9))
 (segment (start 130.863 46.999) (end 130.863 48.929) (width 1) (layer "B.Cu") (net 9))
 (segment (start 145.225 52.925) (end 147.75 55.45) (width 1) (layer "B.Cu") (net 9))
 (segment (start 102.217 80.572) (end 102.217 64.583) (width 1) (layer "B.Cu") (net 18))
 (segment (start 146.639 84.286) (end 145.016 84.286) (width 1) (layer "B.Cu") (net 18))
 (segment (start 102.217 64.583) (end 122.35 44.45) (width 1) (layer "B.Cu") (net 18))
 (segment (start 149.225 50.1) (end 149.225 81.7) (width 1) (layer "B.Cu") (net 18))
 (segment (start 122.35 44.45) (end 143.575 44.45) (width 1) (layer "B.Cu") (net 18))
 (segment (start 143.575 44.45) (end 149.225 50.1) (width 1) (layer "B.Cu") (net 18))
 (segment (start 149.225 81.7) (end 146.639 84.286) (width 1) (layer "B.Cu") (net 18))
 (segment (start 99.677 80.572) (end 99.677 84.702) (width 1) (layer "B.Cu") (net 19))
 (segment (start 99.677 84.702) (end 99.8 84.825) (width 1) (layer "B.Cu") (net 19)))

